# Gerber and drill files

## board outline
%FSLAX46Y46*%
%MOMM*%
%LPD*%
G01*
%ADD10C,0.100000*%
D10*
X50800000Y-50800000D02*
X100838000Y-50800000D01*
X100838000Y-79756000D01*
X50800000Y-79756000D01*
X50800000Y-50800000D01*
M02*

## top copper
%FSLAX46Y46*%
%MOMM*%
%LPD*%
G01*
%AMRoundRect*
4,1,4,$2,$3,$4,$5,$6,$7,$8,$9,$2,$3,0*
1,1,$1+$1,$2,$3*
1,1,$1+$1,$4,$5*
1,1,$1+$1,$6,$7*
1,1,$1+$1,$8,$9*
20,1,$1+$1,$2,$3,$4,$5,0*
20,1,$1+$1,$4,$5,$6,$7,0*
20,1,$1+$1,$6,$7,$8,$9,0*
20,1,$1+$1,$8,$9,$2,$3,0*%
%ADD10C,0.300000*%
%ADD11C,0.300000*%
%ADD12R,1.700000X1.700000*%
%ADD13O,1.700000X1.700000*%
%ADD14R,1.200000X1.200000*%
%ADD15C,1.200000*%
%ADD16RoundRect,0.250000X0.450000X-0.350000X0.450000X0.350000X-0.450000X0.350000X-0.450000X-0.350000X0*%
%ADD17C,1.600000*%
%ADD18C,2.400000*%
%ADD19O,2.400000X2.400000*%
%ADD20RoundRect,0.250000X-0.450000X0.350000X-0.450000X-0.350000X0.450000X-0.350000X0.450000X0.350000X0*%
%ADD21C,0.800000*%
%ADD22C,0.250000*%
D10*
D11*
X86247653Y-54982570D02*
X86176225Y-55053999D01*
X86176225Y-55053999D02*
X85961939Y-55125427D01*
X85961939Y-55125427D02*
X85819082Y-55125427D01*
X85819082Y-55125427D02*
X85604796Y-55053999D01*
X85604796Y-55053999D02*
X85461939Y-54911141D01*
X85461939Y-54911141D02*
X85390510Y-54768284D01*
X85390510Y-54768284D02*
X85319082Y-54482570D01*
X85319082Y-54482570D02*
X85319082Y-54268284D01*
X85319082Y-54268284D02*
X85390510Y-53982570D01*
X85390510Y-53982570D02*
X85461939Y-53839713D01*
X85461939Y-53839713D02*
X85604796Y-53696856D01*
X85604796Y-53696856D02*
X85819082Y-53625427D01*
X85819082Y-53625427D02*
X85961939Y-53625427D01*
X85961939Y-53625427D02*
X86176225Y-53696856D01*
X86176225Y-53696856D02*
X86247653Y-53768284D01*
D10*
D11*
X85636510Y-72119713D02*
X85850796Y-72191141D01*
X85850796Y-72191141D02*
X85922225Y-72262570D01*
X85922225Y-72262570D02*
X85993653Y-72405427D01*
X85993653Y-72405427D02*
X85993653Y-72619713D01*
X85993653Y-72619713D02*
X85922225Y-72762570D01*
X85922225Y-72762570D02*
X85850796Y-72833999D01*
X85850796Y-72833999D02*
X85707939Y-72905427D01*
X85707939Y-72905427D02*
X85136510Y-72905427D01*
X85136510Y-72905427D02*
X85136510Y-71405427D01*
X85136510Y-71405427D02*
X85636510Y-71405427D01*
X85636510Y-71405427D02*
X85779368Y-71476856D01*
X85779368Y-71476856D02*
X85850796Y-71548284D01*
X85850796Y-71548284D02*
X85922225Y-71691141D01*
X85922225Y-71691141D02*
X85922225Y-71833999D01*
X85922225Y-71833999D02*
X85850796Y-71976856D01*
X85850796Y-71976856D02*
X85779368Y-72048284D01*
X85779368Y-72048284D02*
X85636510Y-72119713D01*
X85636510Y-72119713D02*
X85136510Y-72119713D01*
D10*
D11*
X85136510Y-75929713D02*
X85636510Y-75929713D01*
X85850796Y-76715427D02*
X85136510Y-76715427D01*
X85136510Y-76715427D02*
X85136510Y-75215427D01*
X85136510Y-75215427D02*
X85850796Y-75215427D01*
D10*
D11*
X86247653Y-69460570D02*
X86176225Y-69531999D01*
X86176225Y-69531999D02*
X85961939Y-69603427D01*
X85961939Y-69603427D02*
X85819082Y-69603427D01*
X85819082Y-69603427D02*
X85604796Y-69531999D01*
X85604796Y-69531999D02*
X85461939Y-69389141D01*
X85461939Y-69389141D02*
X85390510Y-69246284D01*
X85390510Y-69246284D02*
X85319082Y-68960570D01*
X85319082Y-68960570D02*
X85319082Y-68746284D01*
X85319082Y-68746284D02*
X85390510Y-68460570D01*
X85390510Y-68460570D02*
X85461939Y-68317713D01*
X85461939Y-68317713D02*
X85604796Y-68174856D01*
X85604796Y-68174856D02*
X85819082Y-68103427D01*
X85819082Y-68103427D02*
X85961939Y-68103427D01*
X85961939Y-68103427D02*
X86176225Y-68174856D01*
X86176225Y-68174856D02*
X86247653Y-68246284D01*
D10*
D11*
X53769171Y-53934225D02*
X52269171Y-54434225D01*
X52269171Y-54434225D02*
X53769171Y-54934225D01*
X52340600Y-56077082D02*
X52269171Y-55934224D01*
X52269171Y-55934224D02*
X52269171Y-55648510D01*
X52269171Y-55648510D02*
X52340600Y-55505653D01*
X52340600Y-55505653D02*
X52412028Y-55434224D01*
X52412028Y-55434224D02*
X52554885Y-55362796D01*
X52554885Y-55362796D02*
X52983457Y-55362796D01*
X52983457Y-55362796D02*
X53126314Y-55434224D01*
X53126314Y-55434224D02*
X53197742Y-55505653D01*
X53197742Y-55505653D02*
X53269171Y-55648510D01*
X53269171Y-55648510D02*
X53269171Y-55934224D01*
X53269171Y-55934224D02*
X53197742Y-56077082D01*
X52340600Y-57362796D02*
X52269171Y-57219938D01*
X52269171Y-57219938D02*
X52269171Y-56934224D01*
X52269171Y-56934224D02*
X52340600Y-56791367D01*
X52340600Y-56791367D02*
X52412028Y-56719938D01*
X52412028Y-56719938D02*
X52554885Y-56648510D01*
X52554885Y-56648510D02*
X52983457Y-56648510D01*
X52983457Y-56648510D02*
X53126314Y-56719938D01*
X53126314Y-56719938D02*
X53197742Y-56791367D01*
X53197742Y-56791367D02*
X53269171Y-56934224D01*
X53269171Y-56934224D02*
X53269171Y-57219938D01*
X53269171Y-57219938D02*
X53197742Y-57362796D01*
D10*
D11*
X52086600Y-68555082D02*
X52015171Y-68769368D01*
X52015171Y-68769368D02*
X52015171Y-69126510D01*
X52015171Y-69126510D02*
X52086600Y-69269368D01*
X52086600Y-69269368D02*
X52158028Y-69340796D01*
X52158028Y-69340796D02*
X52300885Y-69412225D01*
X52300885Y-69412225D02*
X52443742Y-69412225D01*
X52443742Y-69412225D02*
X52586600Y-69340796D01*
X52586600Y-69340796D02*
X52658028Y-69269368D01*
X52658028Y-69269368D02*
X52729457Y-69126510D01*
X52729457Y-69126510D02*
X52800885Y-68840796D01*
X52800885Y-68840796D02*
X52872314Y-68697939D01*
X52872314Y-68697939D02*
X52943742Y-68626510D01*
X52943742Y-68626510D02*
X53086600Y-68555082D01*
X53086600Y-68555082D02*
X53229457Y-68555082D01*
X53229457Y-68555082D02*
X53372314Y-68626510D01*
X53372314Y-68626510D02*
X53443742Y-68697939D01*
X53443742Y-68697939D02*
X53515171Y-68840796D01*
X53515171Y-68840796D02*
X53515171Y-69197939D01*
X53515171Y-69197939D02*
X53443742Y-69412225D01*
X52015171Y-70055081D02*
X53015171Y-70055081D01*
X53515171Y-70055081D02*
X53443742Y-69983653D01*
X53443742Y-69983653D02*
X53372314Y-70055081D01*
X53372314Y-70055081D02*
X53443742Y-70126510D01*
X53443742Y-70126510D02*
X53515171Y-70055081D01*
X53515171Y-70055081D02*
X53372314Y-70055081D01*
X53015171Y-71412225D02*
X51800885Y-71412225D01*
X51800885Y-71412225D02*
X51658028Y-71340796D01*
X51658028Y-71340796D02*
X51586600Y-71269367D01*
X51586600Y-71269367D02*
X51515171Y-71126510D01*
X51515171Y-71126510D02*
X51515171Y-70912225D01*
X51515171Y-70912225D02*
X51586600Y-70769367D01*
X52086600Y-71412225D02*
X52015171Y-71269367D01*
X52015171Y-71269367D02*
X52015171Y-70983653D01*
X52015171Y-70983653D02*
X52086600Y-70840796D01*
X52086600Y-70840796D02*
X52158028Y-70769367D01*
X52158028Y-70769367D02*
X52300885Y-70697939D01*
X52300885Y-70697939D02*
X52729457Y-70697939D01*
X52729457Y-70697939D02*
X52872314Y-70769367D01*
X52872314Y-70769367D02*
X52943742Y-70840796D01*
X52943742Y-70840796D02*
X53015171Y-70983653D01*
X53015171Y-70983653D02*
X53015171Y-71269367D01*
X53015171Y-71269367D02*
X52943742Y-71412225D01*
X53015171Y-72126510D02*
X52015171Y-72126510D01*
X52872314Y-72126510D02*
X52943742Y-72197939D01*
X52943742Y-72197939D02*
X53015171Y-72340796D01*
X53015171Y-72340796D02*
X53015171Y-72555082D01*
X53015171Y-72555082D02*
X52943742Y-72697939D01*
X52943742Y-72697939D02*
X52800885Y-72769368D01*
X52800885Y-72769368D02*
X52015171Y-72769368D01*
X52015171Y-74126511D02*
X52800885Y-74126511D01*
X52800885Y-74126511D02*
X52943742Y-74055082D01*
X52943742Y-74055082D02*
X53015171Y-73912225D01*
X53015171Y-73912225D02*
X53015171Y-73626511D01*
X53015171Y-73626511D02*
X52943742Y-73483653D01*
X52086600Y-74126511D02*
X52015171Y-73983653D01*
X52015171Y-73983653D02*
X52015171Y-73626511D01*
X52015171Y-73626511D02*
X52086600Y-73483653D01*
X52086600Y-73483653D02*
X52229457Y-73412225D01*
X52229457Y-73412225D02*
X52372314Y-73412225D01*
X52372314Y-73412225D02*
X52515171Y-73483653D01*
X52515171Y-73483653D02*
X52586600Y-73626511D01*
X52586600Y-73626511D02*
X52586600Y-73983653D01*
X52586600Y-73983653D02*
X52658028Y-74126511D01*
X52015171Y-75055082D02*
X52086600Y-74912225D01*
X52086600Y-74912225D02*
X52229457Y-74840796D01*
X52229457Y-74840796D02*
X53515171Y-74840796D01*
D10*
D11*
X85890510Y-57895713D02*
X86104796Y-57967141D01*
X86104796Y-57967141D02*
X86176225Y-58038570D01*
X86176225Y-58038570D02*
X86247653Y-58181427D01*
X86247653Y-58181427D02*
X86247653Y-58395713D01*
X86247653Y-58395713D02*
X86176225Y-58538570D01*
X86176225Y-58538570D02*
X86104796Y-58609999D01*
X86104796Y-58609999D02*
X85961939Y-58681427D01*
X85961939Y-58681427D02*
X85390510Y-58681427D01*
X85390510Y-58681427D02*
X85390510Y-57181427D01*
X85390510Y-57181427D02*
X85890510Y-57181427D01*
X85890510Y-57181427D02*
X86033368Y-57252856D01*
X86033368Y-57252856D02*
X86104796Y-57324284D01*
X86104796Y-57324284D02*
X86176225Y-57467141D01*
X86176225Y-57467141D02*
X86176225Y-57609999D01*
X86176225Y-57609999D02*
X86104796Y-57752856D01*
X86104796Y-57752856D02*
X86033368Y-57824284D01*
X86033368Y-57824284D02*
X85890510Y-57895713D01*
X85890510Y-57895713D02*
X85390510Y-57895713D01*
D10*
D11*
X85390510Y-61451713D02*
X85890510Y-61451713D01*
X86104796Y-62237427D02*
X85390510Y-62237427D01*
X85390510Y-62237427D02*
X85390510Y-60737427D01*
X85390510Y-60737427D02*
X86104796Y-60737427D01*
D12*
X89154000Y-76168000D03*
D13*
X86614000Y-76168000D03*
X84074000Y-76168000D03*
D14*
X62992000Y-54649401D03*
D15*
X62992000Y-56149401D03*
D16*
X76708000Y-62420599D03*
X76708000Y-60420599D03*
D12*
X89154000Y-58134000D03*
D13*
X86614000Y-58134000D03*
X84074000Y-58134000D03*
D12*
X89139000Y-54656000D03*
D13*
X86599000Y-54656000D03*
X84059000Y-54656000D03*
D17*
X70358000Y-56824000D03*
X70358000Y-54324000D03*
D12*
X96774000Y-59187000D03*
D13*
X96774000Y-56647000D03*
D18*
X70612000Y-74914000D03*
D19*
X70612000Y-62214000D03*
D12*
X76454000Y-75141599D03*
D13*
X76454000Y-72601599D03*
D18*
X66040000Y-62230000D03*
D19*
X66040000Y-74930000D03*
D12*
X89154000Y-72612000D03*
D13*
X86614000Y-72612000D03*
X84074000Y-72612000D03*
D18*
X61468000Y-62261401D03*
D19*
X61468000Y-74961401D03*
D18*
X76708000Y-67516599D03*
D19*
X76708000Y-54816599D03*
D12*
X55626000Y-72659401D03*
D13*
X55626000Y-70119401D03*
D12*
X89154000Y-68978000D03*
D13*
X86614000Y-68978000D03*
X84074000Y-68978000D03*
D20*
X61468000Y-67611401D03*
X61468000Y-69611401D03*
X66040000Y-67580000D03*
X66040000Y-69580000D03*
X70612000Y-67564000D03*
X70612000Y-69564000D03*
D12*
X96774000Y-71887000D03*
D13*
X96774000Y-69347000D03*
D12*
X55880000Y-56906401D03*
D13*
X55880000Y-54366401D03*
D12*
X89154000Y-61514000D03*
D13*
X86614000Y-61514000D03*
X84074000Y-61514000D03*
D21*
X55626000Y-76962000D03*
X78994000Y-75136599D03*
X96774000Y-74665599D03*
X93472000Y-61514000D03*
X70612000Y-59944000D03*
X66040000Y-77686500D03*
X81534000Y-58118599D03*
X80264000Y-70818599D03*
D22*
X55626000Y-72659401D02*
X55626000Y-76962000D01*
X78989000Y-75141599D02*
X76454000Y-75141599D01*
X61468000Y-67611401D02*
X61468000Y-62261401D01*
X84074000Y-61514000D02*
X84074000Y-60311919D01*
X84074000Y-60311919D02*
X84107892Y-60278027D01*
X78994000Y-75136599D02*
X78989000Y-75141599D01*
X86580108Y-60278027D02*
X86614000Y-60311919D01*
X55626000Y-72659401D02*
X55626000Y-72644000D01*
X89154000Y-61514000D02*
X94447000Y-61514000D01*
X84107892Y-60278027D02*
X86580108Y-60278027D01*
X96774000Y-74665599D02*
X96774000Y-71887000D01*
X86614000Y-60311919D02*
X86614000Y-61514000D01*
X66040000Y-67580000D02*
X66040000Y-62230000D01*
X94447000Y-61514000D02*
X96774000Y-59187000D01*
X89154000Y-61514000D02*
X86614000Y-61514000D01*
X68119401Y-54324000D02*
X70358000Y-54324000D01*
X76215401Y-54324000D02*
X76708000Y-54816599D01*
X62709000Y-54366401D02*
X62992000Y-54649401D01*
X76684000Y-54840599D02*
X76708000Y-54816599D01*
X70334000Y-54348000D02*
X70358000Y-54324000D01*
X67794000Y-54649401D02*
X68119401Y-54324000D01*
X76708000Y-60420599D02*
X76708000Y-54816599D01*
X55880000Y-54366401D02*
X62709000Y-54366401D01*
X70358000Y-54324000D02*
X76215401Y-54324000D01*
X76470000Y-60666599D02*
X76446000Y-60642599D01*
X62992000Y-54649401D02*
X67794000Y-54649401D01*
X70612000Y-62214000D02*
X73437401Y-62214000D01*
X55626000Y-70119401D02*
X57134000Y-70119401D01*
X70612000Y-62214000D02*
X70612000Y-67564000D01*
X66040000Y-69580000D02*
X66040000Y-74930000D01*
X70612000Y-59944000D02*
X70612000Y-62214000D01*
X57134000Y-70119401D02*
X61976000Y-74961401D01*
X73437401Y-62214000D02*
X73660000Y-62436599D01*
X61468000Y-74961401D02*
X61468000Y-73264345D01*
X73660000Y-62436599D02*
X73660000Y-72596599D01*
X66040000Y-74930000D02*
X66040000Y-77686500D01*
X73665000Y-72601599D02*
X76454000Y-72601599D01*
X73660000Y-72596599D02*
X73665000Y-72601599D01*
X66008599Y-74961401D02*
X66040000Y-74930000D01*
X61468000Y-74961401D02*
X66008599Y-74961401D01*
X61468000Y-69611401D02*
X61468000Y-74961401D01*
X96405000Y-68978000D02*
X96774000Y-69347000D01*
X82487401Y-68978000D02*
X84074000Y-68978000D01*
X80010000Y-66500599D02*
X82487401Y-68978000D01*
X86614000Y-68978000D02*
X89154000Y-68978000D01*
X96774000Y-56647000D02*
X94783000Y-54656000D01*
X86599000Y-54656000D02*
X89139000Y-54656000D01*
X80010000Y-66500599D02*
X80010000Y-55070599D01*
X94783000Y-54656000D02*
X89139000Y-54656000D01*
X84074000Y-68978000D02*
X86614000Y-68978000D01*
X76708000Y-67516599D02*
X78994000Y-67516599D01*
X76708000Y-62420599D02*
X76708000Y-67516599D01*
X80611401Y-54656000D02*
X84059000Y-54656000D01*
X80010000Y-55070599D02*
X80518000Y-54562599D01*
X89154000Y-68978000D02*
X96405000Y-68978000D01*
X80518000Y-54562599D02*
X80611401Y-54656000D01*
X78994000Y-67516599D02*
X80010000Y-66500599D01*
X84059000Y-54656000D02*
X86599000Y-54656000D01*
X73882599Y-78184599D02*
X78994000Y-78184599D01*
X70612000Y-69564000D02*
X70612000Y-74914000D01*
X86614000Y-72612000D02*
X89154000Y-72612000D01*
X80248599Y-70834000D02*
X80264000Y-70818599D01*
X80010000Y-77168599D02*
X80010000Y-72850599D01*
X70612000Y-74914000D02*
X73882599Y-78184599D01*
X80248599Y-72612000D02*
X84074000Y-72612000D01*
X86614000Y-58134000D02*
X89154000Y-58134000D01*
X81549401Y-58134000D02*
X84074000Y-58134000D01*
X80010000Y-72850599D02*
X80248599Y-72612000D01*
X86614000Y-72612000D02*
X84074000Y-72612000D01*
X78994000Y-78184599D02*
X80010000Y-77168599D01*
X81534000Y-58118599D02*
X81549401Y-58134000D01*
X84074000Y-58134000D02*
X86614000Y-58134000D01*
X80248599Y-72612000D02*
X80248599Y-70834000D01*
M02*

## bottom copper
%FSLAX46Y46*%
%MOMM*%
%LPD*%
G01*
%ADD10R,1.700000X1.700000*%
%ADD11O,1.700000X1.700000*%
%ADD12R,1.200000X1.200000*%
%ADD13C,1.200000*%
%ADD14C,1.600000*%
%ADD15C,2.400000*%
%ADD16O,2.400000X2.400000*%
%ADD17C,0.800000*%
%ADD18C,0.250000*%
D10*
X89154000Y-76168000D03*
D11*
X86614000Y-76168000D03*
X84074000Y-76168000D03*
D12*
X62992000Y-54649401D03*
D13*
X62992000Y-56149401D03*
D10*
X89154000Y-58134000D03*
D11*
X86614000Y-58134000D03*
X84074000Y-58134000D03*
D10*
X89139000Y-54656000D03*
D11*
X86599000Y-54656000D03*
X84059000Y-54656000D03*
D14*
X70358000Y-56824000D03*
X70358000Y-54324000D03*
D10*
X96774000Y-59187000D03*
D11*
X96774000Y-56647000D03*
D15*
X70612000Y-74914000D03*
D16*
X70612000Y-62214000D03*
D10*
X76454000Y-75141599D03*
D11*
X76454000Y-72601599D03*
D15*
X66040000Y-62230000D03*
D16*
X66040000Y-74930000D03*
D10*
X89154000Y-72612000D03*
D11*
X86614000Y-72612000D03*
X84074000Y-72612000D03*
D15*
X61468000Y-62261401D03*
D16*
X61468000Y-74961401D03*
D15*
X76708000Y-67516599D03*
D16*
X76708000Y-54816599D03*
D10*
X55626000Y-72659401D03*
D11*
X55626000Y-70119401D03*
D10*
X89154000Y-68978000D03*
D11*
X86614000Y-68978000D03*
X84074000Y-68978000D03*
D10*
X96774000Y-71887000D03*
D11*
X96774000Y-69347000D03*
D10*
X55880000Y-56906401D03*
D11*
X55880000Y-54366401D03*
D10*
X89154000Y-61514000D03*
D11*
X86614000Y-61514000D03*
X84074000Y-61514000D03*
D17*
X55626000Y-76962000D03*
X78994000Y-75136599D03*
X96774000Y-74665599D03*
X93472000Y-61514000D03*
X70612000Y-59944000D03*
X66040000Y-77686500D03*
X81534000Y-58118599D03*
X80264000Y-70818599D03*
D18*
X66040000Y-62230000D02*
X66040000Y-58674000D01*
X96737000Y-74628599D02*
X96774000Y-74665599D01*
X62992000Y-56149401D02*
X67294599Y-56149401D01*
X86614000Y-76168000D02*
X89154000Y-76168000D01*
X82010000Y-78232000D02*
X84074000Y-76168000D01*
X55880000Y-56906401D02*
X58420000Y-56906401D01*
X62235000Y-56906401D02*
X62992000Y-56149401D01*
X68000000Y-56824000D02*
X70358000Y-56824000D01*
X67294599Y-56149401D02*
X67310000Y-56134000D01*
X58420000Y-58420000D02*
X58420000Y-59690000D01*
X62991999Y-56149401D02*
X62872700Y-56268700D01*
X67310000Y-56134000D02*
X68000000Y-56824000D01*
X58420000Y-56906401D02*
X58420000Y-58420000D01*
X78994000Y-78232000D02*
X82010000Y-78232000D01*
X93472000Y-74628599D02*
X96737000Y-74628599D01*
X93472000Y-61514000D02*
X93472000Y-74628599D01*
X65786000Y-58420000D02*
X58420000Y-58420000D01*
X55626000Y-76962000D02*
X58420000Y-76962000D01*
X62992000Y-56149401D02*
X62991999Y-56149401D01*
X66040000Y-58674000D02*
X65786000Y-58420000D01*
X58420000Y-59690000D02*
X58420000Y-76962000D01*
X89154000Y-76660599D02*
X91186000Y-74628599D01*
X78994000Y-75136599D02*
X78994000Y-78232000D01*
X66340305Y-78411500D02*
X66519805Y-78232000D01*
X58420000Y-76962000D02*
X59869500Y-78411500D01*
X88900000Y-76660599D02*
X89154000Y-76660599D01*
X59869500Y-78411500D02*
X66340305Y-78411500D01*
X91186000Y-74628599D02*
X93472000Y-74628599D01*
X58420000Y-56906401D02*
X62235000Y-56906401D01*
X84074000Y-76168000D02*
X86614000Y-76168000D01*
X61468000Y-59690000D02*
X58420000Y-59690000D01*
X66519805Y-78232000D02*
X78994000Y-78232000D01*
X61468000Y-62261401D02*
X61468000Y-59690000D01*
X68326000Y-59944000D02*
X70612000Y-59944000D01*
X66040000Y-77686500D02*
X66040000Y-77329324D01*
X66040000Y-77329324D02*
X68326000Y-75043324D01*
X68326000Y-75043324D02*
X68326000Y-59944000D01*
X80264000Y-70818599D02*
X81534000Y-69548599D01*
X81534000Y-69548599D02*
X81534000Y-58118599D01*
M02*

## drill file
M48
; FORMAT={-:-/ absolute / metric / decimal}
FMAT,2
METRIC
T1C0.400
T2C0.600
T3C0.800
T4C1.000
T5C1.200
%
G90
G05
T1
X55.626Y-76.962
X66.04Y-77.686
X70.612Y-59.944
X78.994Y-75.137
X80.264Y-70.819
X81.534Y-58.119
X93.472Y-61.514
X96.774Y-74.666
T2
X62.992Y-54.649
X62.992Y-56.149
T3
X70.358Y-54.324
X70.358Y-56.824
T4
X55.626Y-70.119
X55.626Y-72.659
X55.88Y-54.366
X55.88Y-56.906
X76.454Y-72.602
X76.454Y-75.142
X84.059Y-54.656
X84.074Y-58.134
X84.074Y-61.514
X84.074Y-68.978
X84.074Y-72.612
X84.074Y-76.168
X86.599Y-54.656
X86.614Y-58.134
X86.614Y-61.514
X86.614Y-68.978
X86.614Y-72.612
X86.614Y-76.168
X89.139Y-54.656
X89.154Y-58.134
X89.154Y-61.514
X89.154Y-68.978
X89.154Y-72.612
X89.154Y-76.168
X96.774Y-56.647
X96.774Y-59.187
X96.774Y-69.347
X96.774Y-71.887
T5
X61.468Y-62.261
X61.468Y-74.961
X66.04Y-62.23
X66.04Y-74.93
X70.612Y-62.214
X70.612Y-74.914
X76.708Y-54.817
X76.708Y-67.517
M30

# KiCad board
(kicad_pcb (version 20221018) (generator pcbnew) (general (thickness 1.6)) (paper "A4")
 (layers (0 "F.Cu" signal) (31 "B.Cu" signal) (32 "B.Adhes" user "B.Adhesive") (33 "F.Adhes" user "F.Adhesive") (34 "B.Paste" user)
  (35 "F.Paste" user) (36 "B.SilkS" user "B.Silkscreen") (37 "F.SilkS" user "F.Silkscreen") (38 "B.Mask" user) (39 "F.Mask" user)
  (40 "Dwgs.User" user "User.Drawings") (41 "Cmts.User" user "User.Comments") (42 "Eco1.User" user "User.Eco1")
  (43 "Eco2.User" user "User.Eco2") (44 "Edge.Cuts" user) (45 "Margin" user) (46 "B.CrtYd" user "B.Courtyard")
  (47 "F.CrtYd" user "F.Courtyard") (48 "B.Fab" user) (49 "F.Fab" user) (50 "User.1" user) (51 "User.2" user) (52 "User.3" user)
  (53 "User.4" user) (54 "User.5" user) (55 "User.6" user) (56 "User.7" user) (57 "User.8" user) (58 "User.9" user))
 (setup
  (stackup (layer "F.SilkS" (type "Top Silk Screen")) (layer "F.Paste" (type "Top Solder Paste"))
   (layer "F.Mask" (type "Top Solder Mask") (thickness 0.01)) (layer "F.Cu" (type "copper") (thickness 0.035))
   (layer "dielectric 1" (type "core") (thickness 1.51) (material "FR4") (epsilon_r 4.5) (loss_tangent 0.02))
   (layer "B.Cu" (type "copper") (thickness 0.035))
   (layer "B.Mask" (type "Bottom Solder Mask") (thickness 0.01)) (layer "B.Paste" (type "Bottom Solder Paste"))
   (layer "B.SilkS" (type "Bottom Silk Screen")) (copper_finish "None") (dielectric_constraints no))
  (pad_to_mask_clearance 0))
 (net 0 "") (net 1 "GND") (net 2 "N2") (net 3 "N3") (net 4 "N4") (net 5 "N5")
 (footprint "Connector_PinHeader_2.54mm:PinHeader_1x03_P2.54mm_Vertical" (layer "F.Cu") (at 89.154 76.168 -90)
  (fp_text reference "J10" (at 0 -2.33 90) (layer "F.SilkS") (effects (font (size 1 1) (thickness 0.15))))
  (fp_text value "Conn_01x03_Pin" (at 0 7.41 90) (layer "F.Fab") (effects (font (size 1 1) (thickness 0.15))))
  (pad "1" thru_hole rect (at 0 0 270) (size 1.7 1.7) (drill 1) (layers "*.Cu" "*.Mask") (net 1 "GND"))
  (pad "2" thru_hole oval (at 0 2.54 270) (size 1.7 1.7) (drill 1) (layers "*.Cu" "*.Mask") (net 1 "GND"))
  (pad "3" thru_hole oval (at 0 5.08 270) (size 1.7 1.7) (drill 1) (layers "*.Cu" "*.Mask") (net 1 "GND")))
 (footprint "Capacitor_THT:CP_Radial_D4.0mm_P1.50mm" (layer "F.Cu") (at 62.992 54.649401 -90)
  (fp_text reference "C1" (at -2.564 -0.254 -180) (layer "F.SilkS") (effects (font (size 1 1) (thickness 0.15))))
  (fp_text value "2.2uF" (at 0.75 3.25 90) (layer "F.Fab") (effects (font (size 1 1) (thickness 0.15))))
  (pad "1" thru_hole rect (at 0 0 270) (size 1.2 1.2) (drill 0.6) (layers "*.Cu" "*.Mask") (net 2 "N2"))
  (pad "2" thru_hole circle (at 1.5 0 270) (size 1.2 1.2) (drill 0.6) (layers "*.Cu" "*.Mask") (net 1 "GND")))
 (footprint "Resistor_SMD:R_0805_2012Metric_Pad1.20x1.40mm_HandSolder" (layer "F.Cu") (at 76.708 61.420599 90)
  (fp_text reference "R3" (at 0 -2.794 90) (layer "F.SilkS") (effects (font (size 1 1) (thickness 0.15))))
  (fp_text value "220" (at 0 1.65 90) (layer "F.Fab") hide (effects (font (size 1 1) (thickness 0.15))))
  (pad "1" smd roundrect (at -1 0 90) (size 1.2 1.4) (layers "F.Cu" "F.Paste" "F.Mask") (roundrect_rratio 0.208333) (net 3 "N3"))
  (pad "2" smd roundrect (at 1 0 90) (size 1.2 1.4) (layers "F.Cu" "F.Paste" "F.Mask") (roundrect_rratio 0.208333) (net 2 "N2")))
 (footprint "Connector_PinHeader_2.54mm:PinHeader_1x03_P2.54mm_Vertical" (layer "F.Cu") (at 89.154 58.134 -90)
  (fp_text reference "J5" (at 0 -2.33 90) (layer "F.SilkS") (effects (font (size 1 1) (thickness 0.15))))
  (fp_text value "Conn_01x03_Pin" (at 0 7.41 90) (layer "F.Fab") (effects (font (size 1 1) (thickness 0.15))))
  (pad "1" thru_hole rect (at 0 0 270) (size 1.7 1.7) (drill 1) (layers "*.Cu" "*.Mask") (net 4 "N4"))
  (pad "2" thru_hole oval (at 0 2.54 270) (size 1.7 1.7) (drill 1) (layers "*.Cu" "*.Mask") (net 4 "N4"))
  (pad "3" thru_hole oval (at 0 5.08 270) (size 1.7 1.7) (drill 1) (layers "*.Cu" "*.Mask") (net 4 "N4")))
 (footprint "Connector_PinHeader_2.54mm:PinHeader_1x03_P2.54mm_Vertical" (layer "F.Cu") (at 89.139 54.656 -90)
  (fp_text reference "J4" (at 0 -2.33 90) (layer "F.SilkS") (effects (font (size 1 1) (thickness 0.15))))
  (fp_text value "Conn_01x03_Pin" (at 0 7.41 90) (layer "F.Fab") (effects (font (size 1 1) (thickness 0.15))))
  (pad "1" thru_hole rect (at 0 0 270) (size 1.7 1.7) (drill 1) (layers "*.Cu" "*.Mask") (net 3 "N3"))
  (pad "2" thru_hole oval (at 0 2.54 270) (size 1.7 1.7) (drill 1) (layers "*.Cu" "*.Mask") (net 3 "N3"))
  (pad "3" thru_hole oval (at 0 5.08 270) (size 1.7 1.7) (drill 1) (layers "*.Cu" "*.Mask") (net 3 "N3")))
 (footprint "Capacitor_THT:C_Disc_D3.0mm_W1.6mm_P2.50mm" (layer "F.Cu") (at 70.358 56.824 90)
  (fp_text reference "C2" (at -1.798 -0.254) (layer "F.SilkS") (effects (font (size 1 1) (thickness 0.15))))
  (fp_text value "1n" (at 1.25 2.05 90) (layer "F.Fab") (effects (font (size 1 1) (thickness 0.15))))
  (pad "1" thru_hole circle (at 0 0 90) (size 1.6 1.6) (drill 0.8) (layers "*.Cu" "*.Mask") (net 1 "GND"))
  (pad "2" thru_hole circle (at 2.5 0 90) (size 1.6 1.6) (drill 0.8) (layers "*.Cu" "*.Mask") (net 2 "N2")))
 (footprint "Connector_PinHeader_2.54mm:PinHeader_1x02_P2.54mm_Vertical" (layer "F.Cu") (at 96.774 59.187 180)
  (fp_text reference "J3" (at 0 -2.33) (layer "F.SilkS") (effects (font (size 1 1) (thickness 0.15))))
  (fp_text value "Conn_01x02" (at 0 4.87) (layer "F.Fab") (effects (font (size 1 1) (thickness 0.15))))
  (pad "1" thru_hole rect (at 0 0 180) (size 1.7 1.7) (drill 1) (layers "*.Cu" "*.Mask") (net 1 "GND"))
  (pad "2" thru_hole oval (at 0 2.54 180) (size 1.7 1.7) (drill 1) (layers "*.Cu" "*.Mask") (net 3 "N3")))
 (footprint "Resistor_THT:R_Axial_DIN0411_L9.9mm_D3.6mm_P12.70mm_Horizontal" (layer "F.Cu") (at 70.612 74.914 90)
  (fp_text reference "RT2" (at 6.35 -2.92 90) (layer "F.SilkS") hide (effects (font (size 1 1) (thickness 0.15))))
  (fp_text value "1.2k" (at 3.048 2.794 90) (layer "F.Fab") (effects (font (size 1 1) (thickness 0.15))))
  (pad "1" thru_hole circle (at 0 0 90) (size 2.4 2.4) (drill 1.2) (layers "*.Cu" "*.Mask") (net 4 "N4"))
  (pad "2" thru_hole oval (at 12.7 0 90) (size 2.4 2.4) (drill 1.2) (layers "*.Cu" "*.Mask") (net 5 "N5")))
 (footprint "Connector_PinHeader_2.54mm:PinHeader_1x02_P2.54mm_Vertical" (layer "F.Cu") (at 76.454 75.141599 180)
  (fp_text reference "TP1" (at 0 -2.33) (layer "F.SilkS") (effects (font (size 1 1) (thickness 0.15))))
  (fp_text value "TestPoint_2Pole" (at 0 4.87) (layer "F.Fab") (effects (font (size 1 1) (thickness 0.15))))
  (pad "1" thru_hole rect (at 0 0 180) (size 1.7 1.7) (drill 1) (layers "*.Cu" "*.Mask") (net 1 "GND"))
  (pad "2" thru_hole oval (at 0 2.54 180) (size 1.7 1.7) (drill 1) (layers "*.Cu" "*.Mask") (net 5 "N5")))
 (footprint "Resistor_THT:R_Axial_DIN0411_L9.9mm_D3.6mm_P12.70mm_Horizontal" (layer "F.Cu") (at 66.04 62.23 -90)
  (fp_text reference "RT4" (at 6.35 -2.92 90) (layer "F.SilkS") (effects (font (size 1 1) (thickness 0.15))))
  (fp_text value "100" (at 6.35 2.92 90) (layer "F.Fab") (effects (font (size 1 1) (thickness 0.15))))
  (pad "1" thru_hole circle (at 0 0 270) (size 2.4 2.4) (drill 1.2) (layers "*.Cu" "*.Mask") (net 1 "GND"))
  (pad "2" thru_hole oval (at 12.7 0 270) (size 2.4 2.4) (drill 1.2) (layers "*.Cu" "*.Mask") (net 5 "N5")))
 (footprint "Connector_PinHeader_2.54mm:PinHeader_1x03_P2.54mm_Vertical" (layer "F.Cu") (at 89.154 72.612 -90)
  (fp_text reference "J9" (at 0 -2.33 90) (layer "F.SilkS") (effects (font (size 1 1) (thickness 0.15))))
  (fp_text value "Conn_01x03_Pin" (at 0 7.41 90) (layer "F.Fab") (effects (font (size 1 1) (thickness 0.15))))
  (pad "1" thru_hole rect (at 0 0 270) (size 1.7 1.7) (drill 1) (layers "*.Cu" "*.Mask") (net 4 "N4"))
  (pad "2" thru_hole oval (at 0 2.54 270) (size 1.7 1.7) (drill 1) (layers "*.Cu" "*.Mask") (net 4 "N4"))
  (pad "3" thru_hole oval (at 0 5.08 270) (size 1.7 1.7) (drill 1) (layers "*.Cu" "*.Mask") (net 4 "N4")))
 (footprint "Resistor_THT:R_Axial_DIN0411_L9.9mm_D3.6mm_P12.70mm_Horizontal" (layer "F.Cu") (at 61.468 62.261401 -90)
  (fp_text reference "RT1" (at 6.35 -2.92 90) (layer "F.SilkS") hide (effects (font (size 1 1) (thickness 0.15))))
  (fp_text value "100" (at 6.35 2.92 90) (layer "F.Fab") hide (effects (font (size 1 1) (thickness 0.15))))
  (pad "1" thru_hole circle (at 0 0 270) (size 2.4 2.4) (drill 1.2) (layers "*.Cu" "*.Mask") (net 1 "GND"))
  (pad "2" thru_hole oval (at 12.7 0 270) (size 2.4 2.4) (drill 1.2) (layers "*.Cu" "*.Mask") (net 5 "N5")))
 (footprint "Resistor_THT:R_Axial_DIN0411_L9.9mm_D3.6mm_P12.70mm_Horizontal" (layer "F.Cu") (at 76.708 67.516599 90)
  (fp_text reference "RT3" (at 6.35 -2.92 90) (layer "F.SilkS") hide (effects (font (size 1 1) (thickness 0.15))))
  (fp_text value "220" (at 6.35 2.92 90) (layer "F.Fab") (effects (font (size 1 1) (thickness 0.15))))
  (pad "1" thru_hole circle (at 0 0 90) (size 2.4 2.4) (drill 1.2) (layers "*.Cu" "*.Mask") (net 3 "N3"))
  (pad "2" thru_hole oval (at 12.7 0 90) (size 2.4 2.4) (drill 1.2) (layers "*.Cu" "*.Mask") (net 2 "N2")))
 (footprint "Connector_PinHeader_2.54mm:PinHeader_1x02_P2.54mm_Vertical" (layer "F.Cu") (at 55.626 72.659401 180)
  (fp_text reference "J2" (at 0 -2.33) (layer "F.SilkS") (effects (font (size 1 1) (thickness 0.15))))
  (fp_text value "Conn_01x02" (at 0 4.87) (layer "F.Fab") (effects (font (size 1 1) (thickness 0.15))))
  (pad "1" thru_hole rect (at 0 0 180) (size 1.7 1.7) (drill 1) (layers "*.Cu" "*.Mask") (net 1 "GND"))
  (pad "2" thru_hole oval (at 0 2.54 180) (size 1.7 1.7) (drill 1) (layers "*.Cu" "*.Mask") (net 5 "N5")))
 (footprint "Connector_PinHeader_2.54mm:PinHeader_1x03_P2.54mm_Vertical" (layer "F.Cu") (at 89.154 68.978 -90)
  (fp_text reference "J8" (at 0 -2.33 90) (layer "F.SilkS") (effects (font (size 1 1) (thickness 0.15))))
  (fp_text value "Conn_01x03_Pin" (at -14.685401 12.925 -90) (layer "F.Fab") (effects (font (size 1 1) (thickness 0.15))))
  (pad "1" thru_hole rect (at 0 0 270) (size 1.7 1.7) (drill 1) (layers "*.Cu" "*.Mask") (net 3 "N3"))
  (pad "2" thru_hole oval (at 0 2.54 270) (size 1.7 1.7) (drill 1) (layers "*.Cu" "*.Mask") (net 3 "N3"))
  (pad "3" thru_hole oval (at 0 5.08 270) (size 1.7 1.7) (drill 1) (layers "*.Cu" "*.Mask") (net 3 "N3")))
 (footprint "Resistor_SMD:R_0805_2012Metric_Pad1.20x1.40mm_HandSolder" (layer "F.Cu") (at 61.468 68.611401 -90)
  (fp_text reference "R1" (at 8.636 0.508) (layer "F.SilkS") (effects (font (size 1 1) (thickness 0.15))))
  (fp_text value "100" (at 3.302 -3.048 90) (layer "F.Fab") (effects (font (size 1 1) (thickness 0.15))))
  (pad "1" smd roundrect (at -1 0 270) (size 1.2 1.4) (layers "F.Cu" "F.Paste" "F.Mask") (roundrect_rratio 0.208333) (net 1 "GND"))
  (pad "2" smd roundrect (at 1 0 270) (size 1.2 1.4) (layers "F.Cu" "F.Paste" "F.Mask") (roundrect_rratio 0.208333) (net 5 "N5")))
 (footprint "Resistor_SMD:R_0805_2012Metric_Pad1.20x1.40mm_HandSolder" (layer "F.Cu") (at 66.04 68.58 -90)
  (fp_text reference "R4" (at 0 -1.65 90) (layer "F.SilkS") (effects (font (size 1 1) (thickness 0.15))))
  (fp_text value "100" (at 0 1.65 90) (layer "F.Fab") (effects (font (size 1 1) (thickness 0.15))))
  (pad "1" smd roundrect (at -1 0 270) (size 1.2 1.4) (layers "F.Cu" "F.Paste" "F.Mask") (roundrect_rratio 0.208333) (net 1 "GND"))
  (pad "2" smd roundrect (at 1 0 270) (size 1.2 1.4) (layers "F.Cu" "F.Paste" "F.Mask") (roundrect_rratio 0.208333) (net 5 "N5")))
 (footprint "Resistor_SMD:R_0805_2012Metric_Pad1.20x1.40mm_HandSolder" (layer "F.Cu") (at 70.612 68.564 -90)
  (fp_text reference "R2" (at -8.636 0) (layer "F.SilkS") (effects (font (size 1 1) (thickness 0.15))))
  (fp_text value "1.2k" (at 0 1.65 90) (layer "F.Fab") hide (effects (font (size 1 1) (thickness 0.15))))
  (pad "1" smd roundrect (at -1 0 270) (size 1.2 1.4) (layers "F.Cu" "F.Paste" "F.Mask") (roundrect_rratio 0.208333) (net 5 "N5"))
  (pad "2" smd roundrect (at 1 0 270) (size 1.2 1.4) (layers "F.Cu" "F.Paste" "F.Mask") (roundrect_rratio 0.208333) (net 4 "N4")))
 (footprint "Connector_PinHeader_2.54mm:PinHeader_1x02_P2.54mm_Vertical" (layer "F.Cu") (at 96.774 71.887 180)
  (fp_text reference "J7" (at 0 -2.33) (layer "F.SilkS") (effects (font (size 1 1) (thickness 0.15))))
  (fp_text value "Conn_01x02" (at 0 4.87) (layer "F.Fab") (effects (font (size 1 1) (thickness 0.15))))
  (pad "1" thru_hole rect (at 0 0 180) (size 1.7 1.7) (drill 1) (layers "*.Cu" "*.Mask") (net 1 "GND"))
  (pad "2" thru_hole oval (at 0 2.54 180) (size 1.7 1.7) (drill 1) (layers "*.Cu" "*.Mask") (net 3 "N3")))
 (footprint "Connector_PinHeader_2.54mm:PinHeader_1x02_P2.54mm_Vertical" (layer "F.Cu") (at 55.88 56.906401 180)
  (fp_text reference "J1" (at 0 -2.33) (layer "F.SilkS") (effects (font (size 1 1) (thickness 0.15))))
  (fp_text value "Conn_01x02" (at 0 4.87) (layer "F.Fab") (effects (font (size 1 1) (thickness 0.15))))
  (pad "1" thru_hole rect (at 0 0 180) (size 1.7 1.7) (drill 1) (layers "*.Cu" "*.Mask") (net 1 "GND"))
  (pad "2" thru_hole oval (at 0 2.54 180) (size 1.7 1.7) (drill 1) (layers "*.Cu" "*.Mask") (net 2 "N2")))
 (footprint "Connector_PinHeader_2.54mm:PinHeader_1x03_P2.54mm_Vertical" (layer "F.Cu") (at 89.154 61.514 -90)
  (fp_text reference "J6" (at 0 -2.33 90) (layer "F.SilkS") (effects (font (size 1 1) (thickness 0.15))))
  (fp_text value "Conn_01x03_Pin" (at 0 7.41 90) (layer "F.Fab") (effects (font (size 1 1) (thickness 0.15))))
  (pad "1" thru_hole rect (at 0 0 270) (size 1.7 1.7) (drill 1) (layers "*.Cu" "*.Mask") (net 1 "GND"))
  (pad "2" thru_hole oval (at 0 2.54 270) (size 1.7 1.7) (drill 1) (layers "*.Cu" "*.Mask") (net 1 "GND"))
  (pad "3" thru_hole oval (at 0 5.08 270) (size 1.7 1.7) (drill 1) (layers "*.Cu" "*.Mask") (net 1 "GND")))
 (gr_rect (start 50.8 50.8) (end 100.838 79.756) (stroke (width 0.1) (type default)) (fill none) (layer "Edge.Cuts"))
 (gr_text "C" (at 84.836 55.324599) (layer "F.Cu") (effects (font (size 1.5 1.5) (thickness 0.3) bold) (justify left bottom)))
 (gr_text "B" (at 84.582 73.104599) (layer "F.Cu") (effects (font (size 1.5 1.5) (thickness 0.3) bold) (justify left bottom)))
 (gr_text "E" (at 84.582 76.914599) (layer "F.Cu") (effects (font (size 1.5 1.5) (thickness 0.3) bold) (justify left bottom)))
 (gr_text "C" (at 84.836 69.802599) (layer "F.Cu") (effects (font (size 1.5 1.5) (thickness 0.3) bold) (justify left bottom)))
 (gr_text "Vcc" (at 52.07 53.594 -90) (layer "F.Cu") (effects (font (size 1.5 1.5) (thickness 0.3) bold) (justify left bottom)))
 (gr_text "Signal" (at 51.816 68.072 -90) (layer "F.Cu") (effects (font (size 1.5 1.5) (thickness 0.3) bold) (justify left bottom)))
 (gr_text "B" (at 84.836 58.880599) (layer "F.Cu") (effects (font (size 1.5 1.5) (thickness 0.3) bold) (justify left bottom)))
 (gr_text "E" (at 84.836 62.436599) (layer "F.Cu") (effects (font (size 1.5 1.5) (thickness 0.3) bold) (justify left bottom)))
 (segment (start 55.626 72.659401) (end 55.626 76.962) (width 0.25) (layer "F.Cu") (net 1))
 (segment (start 78.989 75.141599) (end 76.454 75.141599) (width 0.25) (layer "F.Cu") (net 1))
 (segment (start 61.468 67.611401) (end 61.468 62.261401) (width 0.25) (layer "F.Cu") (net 1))
 (segment (start 84.074 61.514) (end 84.074 60.311919) (width 0.25) (layer "F.Cu") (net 1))
 (segment (start 84.074 60.311919) (end 84.107892 60.278027) (width 0.25) (layer "F.Cu") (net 1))
 (segment (start 78.994 75.136599) (end 78.989 75.141599) (width 0.25) (layer "F.Cu") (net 1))
 (segment (start 86.580108 60.278027) (end 86.614 60.311919) (width 0.25) (layer "F.Cu") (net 1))
 (segment (start 55.626 72.659401) (end 55.626 72.644) (width 0.25) (layer "F.Cu") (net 1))
 (segment (start 89.154 61.514) (end 94.447 61.514) (width 0.25) (layer "F.Cu") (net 1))
 (segment (start 84.107892 60.278027) (end 86.580108 60.278027) (width 0.25) (layer "F.Cu") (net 1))
 (segment (start 96.774 74.665599) (end 96.774 71.887) (width 0.25) (layer "F.Cu") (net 1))
 (segment (start 86.614 60.311919) (end 86.614 61.514) (width 0.25) (layer "F.Cu") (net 1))
 (segment (start 66.04 67.58) (end 66.04 62.23) (width 0.25) (layer "F.Cu") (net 1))
 (segment (start 94.447 61.514) (end 96.774 59.187) (width 0.25) (layer "F.Cu") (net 1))
 (segment (start 89.154 61.514) (end 86.614 61.514) (width 0.25) (layer "F.Cu") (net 1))
 (via (at 55.626 76.962) (size 0.8) (drill 0.4) (layers "F.Cu" "B.Cu") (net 1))
 (via (at 78.994 75.136599) (size 0.8) (drill 0.4) (layers "F.Cu" "B.Cu") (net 1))
 (via (at 96.774 74.665599) (size 0.8) (drill 0.4) (layers "F.Cu" "B.Cu") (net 1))
 (via (at 93.472 61.514) (size 0.8) (drill 0.4) (layers "F.Cu" "B.Cu") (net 1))
 (segment (start 66.04 62.23) (end 66.04 58.674) (width 0.25) (layer "B.Cu") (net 1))
 (segment (start 96.737 74.628599) (end 96.774 74.665599) (width 0.25) (layer "B.Cu") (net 1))
 (segment (start 62.992 56.149401) (end 67.294599 56.149401) (width 0.25) (layer "B.Cu") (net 1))
 (segment (start 86.614 76.168) (end 89.154 76.168) (width 0.25) (layer "B.Cu") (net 1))
 (segment (start 82.01 78.232) (end 84.074 76.168) (width 0.25) (layer "B.Cu") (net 1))
 (segment (start 55.88 56.906401) (end 58.42 56.906401) (width 0.25) (layer "B.Cu") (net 1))
 (segment (start 62.235 56.906401) (end 62.992 56.149401) (width 0.25) (layer "B.Cu") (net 1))
 (segment (start 68 56.824) (end 70.358 56.824) (width 0.25) (layer "B.Cu") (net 1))
 (segment (start 67.294599 56.149401) (end 67.31 56.134) (width 0.25) (layer "B.Cu") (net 1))
 (segment (start 58.42 58.42) (end 58.42 59.69) (width 0.25) (layer "B.Cu") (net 1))
 (segment (start 62.991999 56.149401) (end 62.8727 56.2687) (width 0.25) (layer "B.Cu") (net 1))
 (segment (start 67.31 56.134) (end 68 56.824) (width 0.25) (layer "B.Cu") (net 1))
 (segment (start 58.42 56.906401) (end 58.42 58.42) (width 0.25) (layer "B.Cu") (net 1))
 (segment (start 78.994 78.232) (end 82.01 78.232) (width 0.25) (layer "B.Cu") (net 1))
 (segment (start 93.472 74.628599) (end 96.737 74.628599) (width 0.25) (layer "B.Cu") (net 1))
 (segment (start 93.472 61.514) (end 93.472 74.628599) (width 0.25) (layer "B.Cu") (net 1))
 (segment (start 65.786 58.42) (end 58.42 58.42) (width 0.25) (layer "B.Cu") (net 1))
 (segment (start 55.626 76.962) (end 58.42 76.962) (width 0.25) (layer "B.Cu") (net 1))
 (segment (start 62.992 56.149401) (end 62.991999 56.149401) (width 0.25) (layer "B.Cu") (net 1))
 (segment (start 66.04 58.674) (end 65.786 58.42) (width 0.25) (layer "B.Cu") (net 1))
 (segment (start 58.42 59.69) (end 58.42 76.962) (width 0.25) (layer "B.Cu") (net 1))
 (segment (start 89.154 76.660599) (end 91.186 74.628599) (width 0.25) (layer "B.Cu") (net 1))
 (segment (start 78.994 75.136599) (end 78.994 78.232) (width 0.25) (layer "B.Cu") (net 1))
 (segment (start 66.340305 78.4115) (end 66.519805 78.232) (width 0.25) (layer "B.Cu") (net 1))
 (segment (start 58.42 76.962) (end 59.8695 78.4115) (width 0.25) (layer "B.Cu") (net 1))
 (segment (start 88.9 76.660599) (end 89.154 76.660599) (width 0.25) (layer "B.Cu") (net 1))
 (segment (start 59.8695 78.4115) (end 66.340305 78.4115) (width 0.25) (layer "B.Cu") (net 1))
 (segment (start 91.186 74.628599) (end 93.472 74.628599) (width 0.25) (layer "B.Cu") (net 1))
 (segment (start 58.42 56.906401) (end 62.235 56.906401) (width 0.25) (layer "B.Cu") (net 1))
 (segment (start 84.074 76.168) (end 86.614 76.168) (width 0.25) (layer "B.Cu") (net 1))
 (segment (start 61.468 59.69) (end 58.42 59.69) (width 0.25) (layer "B.Cu") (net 1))
 (segment (start 66.519805 78.232) (end 78.994 78.232) (width 0.25) (layer "B.Cu") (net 1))
 (segment (start 61.468 62.261401) (end 61.468 59.69) (width 0.25) (layer "B.Cu") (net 1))
 (segment (start 68.119401 54.324) (end 70.358 54.324) (width 0.25) (layer "F.Cu") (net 2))
 (segment (start 76.215401 54.324) (end 76.708 54.816599) (width 0.25) (layer "F.Cu") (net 2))
 (segment (start 62.709 54.366401) (end 62.992 54.649401) (width 0.25) (layer "F.Cu") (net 2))
 (segment (start 76.684 54.840599) (end 76.708 54.816599) (width 0.25) (layer "F.Cu") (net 2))
 (segment (start 70.334 54.348) (end 70.358 54.324) (width 0.25) (layer "F.Cu") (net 2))
 (segment (start 67.794 54.649401) (end 68.119401 54.324) (width 0.25) (layer "F.Cu") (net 2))
 (segment (start 76.708 60.420599) (end 76.708 54.816599) (width 0.25) (layer "F.Cu") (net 2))
 (segment (start 55.88 54.366401) (end 62.709 54.366401) (width 0.25) (layer "F.Cu") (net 2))
 (segment (start 70.358 54.324) (end 76.215401 54.324) (width 0.25) (layer "F.Cu") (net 2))
 (segment (start 76.47 60.666599) (end 76.446 60.642599) (width 0.25) (layer "F.Cu") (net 2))
 (segment (start 62.992 54.649401) (end 67.794 54.649401) (width 0.25) (layer "F.Cu") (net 2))
 (segment (start 70.612 62.214) (end 73.437401 62.214) (width 0.25) (layer "F.Cu") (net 5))
 (segment (start 55.626 70.119401) (end 57.134 70.119401) (width 0.25) (layer "F.Cu") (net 5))
 (segment (start 70.612 62.214) (end 70.612 67.564) (width 0.25) (layer "F.Cu") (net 5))
 (segment (start 66.04 69.58) (end 66.04 74.93) (width 0.25) (layer "F.Cu") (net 5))
 (segment (start 70.612 59.944) (end 70.612 62.214) (width 0.25) (layer "F.Cu") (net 5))
 (segment (start 57.134 70.119401) (end 61.976 74.961401) (width 0.25) (layer "F.Cu") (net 5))
 (segment (start 73.437401 62.214) (end 73.66 62.436599) (width 0.25) (layer "F.Cu") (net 5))
 (segment (start 61.468 74.961401) (end 61.468 73.264345) (width 0.25) (layer "F.Cu") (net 5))
 (segment (start 73.66 62.436599) (end 73.66 72.596599) (width 0.25) (layer "F.Cu") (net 5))
 (segment (start 66.04 74.93) (end 66.04 77.6865) (width 0.25) (layer "F.Cu") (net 5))
 (segment (start 73.665 72.601599) (end 76.454 72.601599) (width 0.25) (layer "F.Cu") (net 5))
 (segment (start 73.66 72.596599) (end 73.665 72.601599) (width 0.25) (layer "F.Cu") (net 5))
 (segment (start 66.008599 74.961401) (end 66.04 74.93) (width 0.25) (layer "F.Cu") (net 5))
 (segment (start 61.468 74.961401) (end 66.008599 74.961401) (width 0.25) (layer "F.Cu") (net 5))
 (segment (start 61.468 69.611401) (end 61.468 74.961401) (width 0.25) (layer "F.Cu") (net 5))
 (via (at 70.612 59.944) (size 0.8) (drill 0.4) (layers "F.Cu" "B.Cu") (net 5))
 (via (at 66.04 77.6865) (size 0.8) (drill 0.4) (layers "F.Cu" "B.Cu") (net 5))
 (segment (start 68.326 59.944) (end 70.612 59.944) (width 0.25) (layer "B.Cu") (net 5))
 (segment (start 66.04 77.6865) (end 66.04 77.329324) (width 0.25) (layer "B.Cu") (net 5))
 (segment (start 66.04 77.329324) (end 68.326 75.043324) (width 0.25) (layer "B.Cu") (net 5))
 (segment (start 68.326 75.043324) (end 68.326 59.944) (width 0.25) (layer "B.Cu") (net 5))
 (segment (start 96.405 68.978) (end 96.774 69.347) (width 0.25) (layer "F.Cu") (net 3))
 (segment (start 82.487401 68.978) (end 84.074 68.978) (width 0.25) (layer "F.Cu") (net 3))
 (segment (start 80.01 66.500599) (end 82.487401 68.978) (width 0.25) (layer "F.Cu") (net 3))
 (segment (start 86.614 68.978) (end 89.154 68.978) (width 0.25) (layer "F.Cu") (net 3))
 (segment (start 96.774 56.647) (end 94.783 54.656) (width 0.25) (layer "F.Cu") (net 3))
 (segment (start 86.599 54.656) (end 89.139 54.656) (width 0.25) (layer "F.Cu") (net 3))
 (segment (start 80.01 66.500599) (end 80.01 55.070599) (width 0.25) (layer "F.Cu") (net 3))
 (segment (start 94.783 54.656) (end 89.139 54.656) (width 0.25) (layer "F.Cu") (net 3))
 (segment (start 84.074 68.978) (end 86.614 68.978) (width 0.25) (layer "F.Cu") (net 3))
 (segment (start 76.708 67.516599) (end 78.994 67.516599) (width 0.25) (layer "F.Cu") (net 3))
 (segment (start 76.708 62.420599) (end 76.708 67.516599) (width 0.25) (layer "F.Cu") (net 3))
 (segment (start 80.611401 54.656) (end 84.059 54.656) (width 0.25) (layer "F.Cu") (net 3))
 (segment (start 80.01 55.070599) (end 80.518 54.562599) (width 0.25) (layer "F.Cu") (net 3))
 (segment (start 89.154 68.978) (end 96.405 68.978) (width 0.25) (layer "F.Cu") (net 3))
 (segment (start 80.518 54.562599) (end 80.611401 54.656) (width 0.25) (layer "F.Cu") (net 3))
 (segment (start 78.994 67.516599) (end 80.01 66.500599) (width 0.25) (layer "F.Cu") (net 3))
 (segment (start 84.059 54.656) (end 86.599 54.656) (width 0.25) (layer "F.Cu") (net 3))
 (segment (start 73.882599 78.184599) (end 78.994 78.184599) (width 0.25) (layer "F.Cu") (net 4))
 (segment (start 70.612 69.564) (end 70.612 74.914) (width 0.25) (layer "F.Cu") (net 4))
 (segment (start 86.614 72.612) (end 89.154 72.612) (width 0.25) (layer "F.Cu") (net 4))
 (segment (start 80.248599 70.834) (end 80.264 70.818599) (width 0.25) (layer "F.Cu") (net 4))
 (segment (start 80.01 77.168599) (end 80.01 72.850599) (width 0.25) (layer "F.Cu") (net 4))
 (segment (start 70.612 74.914) (end 73.882599 78.184599) (width 0.25) (layer "F.Cu") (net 4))
 (segment (start 80.248599 72.612) (end 84.074 72.612) (width 0.25) (layer "F.Cu") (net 4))
 (segment (start 86.614 58.134) (end 89.154 58.134) (width 0.25) (layer "F.Cu") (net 4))
 (segment (start 81.549401 58.134) (end 84.074 58.134) (width 0.25) (layer "F.Cu") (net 4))
 (segment (start 80.01 72.850599) (end 80.248599 72.612) (width 0.25) (layer "F.Cu") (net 4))
 (segment (start 86.614 72.612) (end 84.074 72.612) (width 0.25) (layer "F.Cu") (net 4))
 (segment (start 78.994 78.184599) (end 80.01 77.168599) (width 0.25) (layer "F.Cu") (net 4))
 (segment (start 81.534 58.118599) (end 81.549401 58.134) (width 0.25) (layer "F.Cu") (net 4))
 (segment (start 84.074 58.134) (end 86.614 58.134) (width 0.25) (layer "F.Cu") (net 4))
 (segment (start 80.248599 72.612) (end 80.248599 70.834) (width 0.25) (layer "F.Cu") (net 4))
 (via (at 81.534 58.118599) (size 0.8) (drill 0.4) (layers "F.Cu" "B.Cu") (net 4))
 (via (at 80.264 70.818599) (size 0.8) (drill 0.4) (layers "F.Cu" "B.Cu") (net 4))
 (segment (start 80.264 70.818599) (end 81.534 69.548599) (width 0.25) (layer "B.Cu") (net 4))
 (segment (start 81.534 69.548599) (end 81.534 58.118599) (width 0.25) (layer "B.Cu") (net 4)))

